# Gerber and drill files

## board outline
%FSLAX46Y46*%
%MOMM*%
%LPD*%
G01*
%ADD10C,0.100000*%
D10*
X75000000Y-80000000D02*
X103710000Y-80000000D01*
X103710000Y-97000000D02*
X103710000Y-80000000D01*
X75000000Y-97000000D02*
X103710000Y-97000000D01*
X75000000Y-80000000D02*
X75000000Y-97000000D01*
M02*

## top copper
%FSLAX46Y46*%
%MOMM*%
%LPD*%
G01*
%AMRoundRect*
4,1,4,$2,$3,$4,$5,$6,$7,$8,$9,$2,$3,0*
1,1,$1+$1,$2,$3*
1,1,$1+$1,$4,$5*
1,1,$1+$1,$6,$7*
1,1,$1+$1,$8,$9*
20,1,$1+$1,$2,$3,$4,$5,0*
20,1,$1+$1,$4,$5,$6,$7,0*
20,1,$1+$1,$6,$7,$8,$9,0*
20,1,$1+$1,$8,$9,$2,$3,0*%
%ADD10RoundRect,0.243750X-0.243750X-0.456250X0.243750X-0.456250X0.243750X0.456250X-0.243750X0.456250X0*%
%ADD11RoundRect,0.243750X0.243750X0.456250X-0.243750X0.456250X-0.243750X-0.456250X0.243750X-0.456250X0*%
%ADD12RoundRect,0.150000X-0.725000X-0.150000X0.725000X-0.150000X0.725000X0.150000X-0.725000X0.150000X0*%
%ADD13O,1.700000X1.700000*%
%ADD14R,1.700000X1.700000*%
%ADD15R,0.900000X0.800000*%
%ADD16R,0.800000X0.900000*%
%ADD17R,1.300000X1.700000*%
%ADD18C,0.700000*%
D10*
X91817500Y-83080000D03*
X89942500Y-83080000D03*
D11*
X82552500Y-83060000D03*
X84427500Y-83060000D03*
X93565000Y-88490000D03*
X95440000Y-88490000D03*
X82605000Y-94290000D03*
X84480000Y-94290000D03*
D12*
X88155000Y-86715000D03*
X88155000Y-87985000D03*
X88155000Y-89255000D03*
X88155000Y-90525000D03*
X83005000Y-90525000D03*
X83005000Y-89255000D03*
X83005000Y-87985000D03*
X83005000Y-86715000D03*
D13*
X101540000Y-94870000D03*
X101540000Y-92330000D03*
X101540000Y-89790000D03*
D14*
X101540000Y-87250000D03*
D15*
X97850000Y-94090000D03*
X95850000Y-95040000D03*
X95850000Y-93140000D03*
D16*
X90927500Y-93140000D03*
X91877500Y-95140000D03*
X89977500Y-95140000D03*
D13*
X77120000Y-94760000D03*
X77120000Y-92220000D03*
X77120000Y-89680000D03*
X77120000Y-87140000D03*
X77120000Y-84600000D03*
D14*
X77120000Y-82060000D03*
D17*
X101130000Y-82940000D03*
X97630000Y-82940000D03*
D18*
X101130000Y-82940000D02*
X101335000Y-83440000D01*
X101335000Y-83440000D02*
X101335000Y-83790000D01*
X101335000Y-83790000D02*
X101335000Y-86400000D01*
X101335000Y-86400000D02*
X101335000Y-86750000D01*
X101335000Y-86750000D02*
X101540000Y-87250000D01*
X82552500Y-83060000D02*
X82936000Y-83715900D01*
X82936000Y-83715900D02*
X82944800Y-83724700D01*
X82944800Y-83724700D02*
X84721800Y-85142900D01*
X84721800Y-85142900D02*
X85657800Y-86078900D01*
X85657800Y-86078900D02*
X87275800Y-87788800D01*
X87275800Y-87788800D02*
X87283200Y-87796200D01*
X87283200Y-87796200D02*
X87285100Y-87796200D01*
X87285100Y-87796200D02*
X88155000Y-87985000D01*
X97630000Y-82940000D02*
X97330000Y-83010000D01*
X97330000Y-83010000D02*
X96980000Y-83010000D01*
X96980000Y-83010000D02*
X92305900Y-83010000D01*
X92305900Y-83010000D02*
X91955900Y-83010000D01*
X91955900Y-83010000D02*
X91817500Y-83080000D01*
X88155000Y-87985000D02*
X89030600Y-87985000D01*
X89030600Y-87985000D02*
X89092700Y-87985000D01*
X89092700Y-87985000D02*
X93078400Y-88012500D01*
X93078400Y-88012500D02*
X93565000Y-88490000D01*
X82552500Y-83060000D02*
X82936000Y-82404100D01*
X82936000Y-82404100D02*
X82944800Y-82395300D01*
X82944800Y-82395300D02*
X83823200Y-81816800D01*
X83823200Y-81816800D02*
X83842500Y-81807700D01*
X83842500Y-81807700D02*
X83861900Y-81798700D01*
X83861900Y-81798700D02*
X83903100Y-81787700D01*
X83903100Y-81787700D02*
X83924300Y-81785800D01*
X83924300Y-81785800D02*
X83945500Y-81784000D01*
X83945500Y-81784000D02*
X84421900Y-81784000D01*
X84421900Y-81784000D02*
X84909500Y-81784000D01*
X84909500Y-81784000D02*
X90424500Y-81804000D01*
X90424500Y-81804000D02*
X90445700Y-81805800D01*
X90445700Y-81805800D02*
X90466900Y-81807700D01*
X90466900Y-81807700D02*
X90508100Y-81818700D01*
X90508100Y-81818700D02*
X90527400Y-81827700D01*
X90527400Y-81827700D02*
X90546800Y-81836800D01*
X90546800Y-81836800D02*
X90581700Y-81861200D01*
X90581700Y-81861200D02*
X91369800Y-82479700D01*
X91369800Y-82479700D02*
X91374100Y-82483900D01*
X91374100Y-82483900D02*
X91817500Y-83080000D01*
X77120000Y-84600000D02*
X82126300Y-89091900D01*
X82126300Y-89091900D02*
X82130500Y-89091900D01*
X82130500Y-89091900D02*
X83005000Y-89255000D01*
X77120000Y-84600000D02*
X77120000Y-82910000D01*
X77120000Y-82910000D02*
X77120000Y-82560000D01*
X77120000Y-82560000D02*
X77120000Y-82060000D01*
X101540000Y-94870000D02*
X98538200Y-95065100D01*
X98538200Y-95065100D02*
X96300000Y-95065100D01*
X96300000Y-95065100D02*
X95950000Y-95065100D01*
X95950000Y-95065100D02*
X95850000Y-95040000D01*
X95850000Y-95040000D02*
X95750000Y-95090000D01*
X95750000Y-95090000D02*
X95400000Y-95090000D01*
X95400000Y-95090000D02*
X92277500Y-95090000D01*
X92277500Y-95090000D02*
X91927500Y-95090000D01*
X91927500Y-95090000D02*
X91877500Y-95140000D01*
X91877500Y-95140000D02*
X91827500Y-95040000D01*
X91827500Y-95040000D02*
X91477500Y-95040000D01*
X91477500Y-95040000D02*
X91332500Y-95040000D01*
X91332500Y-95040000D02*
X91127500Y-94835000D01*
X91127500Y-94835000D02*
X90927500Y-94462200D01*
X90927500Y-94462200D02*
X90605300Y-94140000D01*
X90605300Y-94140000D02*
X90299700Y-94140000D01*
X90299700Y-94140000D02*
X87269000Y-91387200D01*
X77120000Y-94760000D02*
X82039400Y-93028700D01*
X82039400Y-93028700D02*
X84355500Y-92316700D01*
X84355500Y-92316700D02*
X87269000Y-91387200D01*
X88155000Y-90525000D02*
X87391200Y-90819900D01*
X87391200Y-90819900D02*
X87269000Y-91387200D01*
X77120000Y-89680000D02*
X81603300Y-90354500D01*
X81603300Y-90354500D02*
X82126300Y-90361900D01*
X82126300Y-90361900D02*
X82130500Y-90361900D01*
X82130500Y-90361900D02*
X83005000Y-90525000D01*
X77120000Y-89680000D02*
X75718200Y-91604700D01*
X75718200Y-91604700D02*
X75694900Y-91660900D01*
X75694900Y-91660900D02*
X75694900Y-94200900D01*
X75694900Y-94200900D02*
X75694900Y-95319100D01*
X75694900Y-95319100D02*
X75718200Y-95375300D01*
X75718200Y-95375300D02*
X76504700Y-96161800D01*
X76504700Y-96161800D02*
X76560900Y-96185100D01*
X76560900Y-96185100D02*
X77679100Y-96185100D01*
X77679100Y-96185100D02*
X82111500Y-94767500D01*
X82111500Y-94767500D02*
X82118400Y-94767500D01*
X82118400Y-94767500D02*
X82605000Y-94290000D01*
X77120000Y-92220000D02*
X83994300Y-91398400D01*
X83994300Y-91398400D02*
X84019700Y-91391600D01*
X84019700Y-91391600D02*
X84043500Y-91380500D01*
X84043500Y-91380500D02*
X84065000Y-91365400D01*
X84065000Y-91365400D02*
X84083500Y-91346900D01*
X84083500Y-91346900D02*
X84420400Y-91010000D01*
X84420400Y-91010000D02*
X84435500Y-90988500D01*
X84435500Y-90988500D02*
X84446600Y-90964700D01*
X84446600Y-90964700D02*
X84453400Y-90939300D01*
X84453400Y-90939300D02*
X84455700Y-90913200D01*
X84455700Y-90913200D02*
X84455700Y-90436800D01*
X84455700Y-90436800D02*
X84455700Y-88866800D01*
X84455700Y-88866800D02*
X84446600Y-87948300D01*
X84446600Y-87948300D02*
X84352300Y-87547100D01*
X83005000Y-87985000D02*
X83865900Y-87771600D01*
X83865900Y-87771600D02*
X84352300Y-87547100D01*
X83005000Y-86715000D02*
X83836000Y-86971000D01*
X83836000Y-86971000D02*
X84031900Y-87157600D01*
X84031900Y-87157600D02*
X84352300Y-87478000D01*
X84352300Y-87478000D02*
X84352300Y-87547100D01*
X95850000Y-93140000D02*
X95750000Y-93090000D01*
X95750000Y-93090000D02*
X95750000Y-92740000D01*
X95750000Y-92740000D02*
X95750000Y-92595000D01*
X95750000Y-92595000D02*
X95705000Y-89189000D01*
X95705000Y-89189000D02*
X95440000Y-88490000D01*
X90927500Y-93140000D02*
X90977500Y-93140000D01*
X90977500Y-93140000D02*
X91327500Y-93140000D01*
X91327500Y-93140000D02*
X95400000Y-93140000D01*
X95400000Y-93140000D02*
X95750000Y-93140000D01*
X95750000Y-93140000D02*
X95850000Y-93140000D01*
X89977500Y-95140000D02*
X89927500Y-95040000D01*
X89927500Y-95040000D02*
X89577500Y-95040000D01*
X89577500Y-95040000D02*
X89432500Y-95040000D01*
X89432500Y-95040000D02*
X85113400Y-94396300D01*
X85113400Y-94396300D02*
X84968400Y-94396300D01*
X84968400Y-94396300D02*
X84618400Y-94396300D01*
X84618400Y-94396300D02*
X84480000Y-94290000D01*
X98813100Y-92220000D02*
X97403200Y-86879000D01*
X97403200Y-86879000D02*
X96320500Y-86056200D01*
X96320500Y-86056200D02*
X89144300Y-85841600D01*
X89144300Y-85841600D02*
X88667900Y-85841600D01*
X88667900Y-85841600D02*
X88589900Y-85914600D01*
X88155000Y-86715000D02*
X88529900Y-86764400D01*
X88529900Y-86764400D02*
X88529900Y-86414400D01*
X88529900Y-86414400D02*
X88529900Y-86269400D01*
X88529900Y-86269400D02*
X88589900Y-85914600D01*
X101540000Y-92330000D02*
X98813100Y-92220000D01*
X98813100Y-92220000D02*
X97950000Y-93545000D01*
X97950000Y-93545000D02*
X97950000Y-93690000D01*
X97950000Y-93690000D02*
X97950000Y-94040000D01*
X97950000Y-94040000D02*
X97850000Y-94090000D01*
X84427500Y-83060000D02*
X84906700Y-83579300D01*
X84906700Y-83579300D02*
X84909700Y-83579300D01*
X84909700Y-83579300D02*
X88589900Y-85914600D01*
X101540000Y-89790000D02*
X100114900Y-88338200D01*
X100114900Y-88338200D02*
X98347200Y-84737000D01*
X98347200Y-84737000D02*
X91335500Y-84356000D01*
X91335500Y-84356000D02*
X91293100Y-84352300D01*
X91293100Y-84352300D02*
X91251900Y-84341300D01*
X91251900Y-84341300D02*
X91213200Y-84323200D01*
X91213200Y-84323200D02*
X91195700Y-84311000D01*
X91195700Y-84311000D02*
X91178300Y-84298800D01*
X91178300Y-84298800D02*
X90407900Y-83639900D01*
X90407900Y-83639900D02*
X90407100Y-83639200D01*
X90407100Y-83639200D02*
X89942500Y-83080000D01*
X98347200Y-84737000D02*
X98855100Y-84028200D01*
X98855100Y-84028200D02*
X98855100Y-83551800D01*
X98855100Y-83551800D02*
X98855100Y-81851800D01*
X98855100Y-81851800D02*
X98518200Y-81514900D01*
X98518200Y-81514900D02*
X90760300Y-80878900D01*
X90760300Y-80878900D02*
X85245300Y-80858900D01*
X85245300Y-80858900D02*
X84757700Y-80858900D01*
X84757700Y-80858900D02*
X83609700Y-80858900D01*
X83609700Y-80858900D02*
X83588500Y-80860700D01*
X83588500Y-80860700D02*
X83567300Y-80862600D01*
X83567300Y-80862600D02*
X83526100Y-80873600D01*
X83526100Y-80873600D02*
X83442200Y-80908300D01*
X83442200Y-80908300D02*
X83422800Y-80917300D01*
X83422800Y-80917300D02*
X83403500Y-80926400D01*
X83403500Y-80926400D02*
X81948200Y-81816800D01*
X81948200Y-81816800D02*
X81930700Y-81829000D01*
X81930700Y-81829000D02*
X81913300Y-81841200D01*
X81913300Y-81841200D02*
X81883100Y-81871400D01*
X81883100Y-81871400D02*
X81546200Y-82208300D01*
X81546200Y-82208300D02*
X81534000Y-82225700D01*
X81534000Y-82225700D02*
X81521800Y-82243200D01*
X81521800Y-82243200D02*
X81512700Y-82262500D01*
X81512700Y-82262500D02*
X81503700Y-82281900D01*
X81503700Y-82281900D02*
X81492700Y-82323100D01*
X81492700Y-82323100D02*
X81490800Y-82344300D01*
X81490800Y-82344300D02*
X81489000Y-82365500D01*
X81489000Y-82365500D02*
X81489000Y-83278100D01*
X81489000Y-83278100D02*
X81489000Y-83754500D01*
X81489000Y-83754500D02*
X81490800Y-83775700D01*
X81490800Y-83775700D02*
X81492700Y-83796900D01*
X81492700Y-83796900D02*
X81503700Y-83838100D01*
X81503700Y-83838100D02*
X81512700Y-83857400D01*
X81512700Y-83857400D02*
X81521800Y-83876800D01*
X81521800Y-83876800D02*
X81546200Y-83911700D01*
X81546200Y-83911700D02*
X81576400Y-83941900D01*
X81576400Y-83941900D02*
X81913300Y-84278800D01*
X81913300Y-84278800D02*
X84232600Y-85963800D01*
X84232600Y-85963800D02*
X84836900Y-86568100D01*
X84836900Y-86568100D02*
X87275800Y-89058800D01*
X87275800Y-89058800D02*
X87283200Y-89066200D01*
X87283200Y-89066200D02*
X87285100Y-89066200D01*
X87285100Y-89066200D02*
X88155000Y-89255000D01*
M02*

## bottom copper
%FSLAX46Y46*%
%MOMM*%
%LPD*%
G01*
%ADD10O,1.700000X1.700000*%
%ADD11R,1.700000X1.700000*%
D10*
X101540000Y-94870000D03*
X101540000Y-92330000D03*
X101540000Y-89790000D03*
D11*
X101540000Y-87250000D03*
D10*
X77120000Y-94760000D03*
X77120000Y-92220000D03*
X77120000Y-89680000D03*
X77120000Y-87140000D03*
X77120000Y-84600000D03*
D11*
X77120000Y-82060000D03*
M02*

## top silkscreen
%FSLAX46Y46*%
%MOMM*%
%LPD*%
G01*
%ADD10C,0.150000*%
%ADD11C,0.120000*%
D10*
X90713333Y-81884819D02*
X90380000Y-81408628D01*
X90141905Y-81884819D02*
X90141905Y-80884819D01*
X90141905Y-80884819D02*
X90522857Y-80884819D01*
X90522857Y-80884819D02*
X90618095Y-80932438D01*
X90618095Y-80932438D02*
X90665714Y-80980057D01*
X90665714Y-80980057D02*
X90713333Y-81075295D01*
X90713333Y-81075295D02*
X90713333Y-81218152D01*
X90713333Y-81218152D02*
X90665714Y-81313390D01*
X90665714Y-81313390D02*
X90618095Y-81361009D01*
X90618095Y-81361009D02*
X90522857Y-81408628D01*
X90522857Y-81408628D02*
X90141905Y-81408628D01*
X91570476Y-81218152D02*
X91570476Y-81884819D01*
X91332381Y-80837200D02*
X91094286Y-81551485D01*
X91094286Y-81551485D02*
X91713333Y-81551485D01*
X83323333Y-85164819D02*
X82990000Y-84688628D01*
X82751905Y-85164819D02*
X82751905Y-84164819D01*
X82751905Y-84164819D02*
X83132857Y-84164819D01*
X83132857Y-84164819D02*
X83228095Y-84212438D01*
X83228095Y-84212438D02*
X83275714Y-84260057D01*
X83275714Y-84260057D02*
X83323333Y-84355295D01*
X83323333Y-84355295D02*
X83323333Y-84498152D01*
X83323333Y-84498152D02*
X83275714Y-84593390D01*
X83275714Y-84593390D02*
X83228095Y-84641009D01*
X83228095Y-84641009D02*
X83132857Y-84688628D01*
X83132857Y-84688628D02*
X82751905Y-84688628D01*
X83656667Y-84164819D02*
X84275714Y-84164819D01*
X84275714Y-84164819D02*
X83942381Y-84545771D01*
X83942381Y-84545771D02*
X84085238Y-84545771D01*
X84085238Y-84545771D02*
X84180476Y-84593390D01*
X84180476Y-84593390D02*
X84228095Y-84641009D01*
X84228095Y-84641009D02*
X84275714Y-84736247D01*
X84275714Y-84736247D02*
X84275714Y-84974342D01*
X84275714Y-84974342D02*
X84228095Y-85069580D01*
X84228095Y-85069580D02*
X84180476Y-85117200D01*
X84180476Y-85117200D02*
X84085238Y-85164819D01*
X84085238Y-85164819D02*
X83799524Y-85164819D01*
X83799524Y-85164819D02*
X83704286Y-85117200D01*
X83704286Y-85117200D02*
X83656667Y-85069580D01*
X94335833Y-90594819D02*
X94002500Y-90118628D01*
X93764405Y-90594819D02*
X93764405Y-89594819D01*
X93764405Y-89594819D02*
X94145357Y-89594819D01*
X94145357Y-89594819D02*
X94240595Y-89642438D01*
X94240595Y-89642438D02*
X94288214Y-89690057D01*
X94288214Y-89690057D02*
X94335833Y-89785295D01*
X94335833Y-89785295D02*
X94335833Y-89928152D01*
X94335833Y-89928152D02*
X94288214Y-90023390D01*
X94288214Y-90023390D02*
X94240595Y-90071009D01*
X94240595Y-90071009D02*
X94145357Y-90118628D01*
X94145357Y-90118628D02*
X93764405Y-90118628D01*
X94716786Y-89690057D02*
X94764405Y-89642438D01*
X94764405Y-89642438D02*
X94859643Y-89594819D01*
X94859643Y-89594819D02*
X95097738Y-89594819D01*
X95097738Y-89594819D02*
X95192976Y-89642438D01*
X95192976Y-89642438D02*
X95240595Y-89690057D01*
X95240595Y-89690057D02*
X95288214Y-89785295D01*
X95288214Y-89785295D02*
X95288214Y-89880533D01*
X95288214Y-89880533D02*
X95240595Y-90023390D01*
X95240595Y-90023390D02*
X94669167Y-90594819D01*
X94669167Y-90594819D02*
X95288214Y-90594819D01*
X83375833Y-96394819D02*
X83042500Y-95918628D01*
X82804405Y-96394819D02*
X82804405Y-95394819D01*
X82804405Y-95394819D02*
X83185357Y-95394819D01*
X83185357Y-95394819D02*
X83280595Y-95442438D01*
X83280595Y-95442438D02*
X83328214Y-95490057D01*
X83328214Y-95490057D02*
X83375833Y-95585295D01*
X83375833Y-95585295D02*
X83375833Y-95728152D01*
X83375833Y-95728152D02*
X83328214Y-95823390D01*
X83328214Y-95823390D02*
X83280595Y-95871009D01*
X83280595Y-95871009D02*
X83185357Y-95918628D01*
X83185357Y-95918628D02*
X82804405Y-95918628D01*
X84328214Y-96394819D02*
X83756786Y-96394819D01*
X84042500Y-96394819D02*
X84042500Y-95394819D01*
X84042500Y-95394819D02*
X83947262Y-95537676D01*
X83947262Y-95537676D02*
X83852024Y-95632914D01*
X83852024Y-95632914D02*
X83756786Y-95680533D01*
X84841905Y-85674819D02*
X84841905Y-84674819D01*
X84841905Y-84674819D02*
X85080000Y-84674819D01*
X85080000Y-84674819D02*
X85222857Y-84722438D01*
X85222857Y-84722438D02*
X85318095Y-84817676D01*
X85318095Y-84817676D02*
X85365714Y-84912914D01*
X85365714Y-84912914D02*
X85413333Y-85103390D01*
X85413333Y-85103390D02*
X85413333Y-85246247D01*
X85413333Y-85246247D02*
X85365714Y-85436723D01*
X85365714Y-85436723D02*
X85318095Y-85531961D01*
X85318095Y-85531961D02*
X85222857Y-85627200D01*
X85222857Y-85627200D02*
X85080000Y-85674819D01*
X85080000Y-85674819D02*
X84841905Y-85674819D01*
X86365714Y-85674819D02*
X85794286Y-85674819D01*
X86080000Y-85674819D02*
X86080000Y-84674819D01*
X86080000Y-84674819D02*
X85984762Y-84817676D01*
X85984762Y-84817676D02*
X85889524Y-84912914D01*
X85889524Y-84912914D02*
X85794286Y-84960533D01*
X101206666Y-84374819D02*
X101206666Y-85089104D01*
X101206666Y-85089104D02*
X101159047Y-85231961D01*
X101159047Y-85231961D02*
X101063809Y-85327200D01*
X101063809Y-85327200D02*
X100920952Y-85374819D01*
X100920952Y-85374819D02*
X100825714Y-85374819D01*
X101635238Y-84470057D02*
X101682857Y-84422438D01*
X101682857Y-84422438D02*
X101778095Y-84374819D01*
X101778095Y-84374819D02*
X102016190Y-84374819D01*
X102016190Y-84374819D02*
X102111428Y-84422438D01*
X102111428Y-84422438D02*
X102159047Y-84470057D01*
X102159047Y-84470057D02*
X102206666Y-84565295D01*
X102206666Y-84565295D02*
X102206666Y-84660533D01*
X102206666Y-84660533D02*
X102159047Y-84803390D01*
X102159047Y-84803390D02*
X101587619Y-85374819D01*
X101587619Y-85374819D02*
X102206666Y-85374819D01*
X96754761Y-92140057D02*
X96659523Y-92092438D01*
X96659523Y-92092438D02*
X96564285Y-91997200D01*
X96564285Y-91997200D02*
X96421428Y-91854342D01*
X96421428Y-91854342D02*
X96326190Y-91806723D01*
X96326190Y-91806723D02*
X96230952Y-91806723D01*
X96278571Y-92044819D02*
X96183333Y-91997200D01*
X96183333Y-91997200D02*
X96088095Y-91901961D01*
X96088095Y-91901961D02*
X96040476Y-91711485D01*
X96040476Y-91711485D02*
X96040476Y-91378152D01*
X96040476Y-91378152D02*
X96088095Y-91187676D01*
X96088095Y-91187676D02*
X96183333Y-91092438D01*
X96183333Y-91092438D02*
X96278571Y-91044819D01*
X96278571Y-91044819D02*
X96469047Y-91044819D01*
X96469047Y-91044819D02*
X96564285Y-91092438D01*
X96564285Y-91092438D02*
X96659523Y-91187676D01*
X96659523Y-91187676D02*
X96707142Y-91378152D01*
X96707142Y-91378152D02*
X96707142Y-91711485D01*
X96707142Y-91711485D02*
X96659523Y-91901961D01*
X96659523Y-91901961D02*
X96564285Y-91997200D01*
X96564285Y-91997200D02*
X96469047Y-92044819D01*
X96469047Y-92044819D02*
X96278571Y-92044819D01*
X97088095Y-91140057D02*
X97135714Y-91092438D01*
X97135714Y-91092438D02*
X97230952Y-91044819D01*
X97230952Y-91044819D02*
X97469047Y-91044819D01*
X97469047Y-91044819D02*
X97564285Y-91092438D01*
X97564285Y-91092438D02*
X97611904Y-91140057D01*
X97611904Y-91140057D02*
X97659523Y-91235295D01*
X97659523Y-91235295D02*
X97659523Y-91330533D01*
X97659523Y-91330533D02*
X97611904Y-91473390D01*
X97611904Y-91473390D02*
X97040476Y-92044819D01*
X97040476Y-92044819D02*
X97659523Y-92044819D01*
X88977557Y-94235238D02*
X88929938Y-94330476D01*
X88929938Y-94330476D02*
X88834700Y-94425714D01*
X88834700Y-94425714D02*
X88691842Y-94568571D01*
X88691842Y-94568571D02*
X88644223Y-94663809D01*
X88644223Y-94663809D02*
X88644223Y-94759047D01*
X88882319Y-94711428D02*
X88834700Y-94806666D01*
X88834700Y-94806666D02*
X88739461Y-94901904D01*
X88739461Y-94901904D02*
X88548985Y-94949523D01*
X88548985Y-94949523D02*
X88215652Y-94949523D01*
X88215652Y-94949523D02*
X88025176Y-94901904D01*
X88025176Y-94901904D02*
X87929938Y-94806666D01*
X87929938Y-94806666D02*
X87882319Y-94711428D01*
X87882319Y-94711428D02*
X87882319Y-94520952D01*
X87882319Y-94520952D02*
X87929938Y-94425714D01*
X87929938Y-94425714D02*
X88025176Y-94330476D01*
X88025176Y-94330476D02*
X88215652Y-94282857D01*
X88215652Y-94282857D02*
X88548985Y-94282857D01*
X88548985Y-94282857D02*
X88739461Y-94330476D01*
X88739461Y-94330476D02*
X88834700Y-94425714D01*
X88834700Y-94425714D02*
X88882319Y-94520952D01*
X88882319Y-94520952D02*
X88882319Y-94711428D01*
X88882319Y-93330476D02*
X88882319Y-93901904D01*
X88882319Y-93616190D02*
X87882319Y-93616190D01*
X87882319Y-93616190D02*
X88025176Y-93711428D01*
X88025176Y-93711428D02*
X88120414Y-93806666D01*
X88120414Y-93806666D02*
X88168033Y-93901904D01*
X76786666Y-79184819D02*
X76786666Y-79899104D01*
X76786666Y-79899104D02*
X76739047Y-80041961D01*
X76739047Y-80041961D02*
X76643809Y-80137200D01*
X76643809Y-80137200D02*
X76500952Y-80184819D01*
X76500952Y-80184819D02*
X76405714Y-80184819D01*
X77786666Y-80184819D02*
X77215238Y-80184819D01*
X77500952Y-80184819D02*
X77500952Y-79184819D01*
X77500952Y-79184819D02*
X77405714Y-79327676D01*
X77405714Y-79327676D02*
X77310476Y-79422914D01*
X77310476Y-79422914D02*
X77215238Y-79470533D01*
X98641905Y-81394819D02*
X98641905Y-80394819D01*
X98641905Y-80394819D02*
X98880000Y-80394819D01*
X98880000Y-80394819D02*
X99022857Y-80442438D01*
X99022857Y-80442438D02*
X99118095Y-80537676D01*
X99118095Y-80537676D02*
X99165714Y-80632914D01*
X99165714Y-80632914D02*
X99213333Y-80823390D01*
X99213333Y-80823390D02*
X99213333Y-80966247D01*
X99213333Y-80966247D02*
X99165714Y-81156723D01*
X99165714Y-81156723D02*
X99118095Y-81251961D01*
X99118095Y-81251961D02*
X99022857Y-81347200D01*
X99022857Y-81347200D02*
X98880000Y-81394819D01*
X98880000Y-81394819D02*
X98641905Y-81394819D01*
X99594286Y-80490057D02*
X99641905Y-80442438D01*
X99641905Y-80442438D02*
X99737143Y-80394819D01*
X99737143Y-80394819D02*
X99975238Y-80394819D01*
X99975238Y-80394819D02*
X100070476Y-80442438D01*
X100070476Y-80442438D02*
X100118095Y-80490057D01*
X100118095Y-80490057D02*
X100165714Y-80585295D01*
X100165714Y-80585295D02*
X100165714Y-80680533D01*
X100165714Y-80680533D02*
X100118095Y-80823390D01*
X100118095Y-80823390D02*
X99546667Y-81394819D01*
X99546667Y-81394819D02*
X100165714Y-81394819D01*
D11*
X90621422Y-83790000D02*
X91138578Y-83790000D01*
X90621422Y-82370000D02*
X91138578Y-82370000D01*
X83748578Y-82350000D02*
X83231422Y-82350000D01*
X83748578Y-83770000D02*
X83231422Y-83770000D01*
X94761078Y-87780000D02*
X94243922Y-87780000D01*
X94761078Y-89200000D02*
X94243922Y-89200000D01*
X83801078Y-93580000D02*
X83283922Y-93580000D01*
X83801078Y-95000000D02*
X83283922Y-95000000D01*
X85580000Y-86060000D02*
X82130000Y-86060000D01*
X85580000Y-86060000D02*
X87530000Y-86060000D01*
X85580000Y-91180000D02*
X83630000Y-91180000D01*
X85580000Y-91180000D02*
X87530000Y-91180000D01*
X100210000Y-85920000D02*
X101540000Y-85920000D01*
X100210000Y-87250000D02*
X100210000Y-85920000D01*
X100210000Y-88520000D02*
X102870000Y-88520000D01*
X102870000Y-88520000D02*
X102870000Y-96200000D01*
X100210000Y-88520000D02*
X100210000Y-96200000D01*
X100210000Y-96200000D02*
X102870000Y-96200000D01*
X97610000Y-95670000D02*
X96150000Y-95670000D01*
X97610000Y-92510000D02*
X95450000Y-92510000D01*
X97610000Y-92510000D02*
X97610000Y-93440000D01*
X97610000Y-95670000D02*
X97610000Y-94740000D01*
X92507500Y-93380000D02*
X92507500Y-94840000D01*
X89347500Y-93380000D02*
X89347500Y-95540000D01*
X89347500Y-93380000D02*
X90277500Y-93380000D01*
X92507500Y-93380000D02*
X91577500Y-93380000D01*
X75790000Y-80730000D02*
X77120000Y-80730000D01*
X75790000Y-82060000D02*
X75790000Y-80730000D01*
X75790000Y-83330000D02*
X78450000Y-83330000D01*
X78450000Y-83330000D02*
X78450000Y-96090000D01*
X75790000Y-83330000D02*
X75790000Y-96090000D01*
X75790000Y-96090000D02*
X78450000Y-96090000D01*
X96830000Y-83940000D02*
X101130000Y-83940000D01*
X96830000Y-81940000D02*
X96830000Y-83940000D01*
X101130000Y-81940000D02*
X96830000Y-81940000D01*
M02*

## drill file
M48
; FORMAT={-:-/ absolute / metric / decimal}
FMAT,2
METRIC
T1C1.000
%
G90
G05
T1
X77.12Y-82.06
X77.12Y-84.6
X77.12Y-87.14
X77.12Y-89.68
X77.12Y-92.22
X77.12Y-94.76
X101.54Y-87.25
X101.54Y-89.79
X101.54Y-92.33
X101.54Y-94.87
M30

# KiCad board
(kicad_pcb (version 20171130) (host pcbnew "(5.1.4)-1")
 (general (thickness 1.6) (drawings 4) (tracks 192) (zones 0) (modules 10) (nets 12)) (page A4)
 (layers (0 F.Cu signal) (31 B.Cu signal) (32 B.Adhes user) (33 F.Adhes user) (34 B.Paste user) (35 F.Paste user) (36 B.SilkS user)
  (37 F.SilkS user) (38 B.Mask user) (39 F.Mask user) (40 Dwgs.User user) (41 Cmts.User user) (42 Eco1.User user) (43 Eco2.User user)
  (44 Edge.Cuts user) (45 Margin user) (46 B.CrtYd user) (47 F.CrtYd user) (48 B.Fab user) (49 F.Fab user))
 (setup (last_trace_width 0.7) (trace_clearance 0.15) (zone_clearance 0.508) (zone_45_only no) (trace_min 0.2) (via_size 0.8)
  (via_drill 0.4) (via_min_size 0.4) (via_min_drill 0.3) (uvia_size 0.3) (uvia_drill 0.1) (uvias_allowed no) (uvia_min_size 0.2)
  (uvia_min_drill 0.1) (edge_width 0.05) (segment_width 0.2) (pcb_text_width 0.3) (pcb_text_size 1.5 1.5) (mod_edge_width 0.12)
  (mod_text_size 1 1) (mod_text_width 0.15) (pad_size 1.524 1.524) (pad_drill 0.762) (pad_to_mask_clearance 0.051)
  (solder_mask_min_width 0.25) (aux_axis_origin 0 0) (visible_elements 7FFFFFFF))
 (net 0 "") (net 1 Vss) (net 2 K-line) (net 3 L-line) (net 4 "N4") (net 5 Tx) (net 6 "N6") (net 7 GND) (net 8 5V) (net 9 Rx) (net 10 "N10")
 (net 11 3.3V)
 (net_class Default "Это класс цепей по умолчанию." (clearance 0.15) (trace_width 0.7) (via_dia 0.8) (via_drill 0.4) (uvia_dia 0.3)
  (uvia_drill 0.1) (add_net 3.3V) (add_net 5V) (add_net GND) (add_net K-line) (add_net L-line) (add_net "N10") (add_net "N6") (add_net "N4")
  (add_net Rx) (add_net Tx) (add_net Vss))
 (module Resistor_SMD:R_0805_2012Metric (layer F.Cu) (at 90.88 83.08)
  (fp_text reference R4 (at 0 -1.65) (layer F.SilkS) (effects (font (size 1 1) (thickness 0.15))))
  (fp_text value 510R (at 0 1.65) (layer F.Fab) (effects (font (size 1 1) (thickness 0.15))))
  (fp_line (start -0.258578 0.71) (end 0.258578 0.71) (layer F.SilkS) (width 0.12))
  (fp_line (start -0.258578 -0.71) (end 0.258578 -0.71) (layer F.SilkS) (width 0.12))
  (pad 2 smd roundrect (at 0.9375 0) (size 0.975 1.4) (layers F.Cu F.Paste F.Mask) (roundrect_rratio 0.25) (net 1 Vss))
  (pad 1 smd roundrect (at -0.9375 0) (size 0.975 1.4) (layers F.Cu F.Paste F.Mask) (roundrect_rratio 0.25) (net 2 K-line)))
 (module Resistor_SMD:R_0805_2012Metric (layer F.Cu) (at 83.49 83.06 180)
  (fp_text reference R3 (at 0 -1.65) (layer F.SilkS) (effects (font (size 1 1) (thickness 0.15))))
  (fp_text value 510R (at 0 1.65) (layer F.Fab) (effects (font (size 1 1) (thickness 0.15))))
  (fp_line (start -0.258578 0.71) (end 0.258578 0.71) (layer F.SilkS) (width 0.12))
  (fp_line (start -0.258578 -0.71) (end 0.258578 -0.71) (layer F.SilkS) (width 0.12))
  (pad 2 smd roundrect (at 0.9375 0 180) (size 0.975 1.4) (layers F.Cu F.Paste F.Mask) (roundrect_rratio 0.25) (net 1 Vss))
  (pad 1 smd roundrect (at -0.9375 0 180) (size 0.975 1.4) (layers F.Cu F.Paste F.Mask) (roundrect_rratio 0.25) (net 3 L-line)))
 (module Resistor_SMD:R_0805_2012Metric (layer F.Cu) (at 94.5025 88.49 180)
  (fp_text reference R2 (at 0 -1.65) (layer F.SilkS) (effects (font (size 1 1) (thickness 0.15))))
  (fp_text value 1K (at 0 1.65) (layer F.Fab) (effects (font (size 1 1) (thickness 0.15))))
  (fp_line (start -0.258578 0.71) (end 0.258578 0.71) (layer F.SilkS) (width 0.12))
  (fp_line (start -0.258578 -0.71) (end 0.258578 -0.71) (layer F.SilkS) (width 0.12))
  (pad 2 smd roundrect (at 0.9375 0 180) (size 0.975 1.4) (layers F.Cu F.Paste F.Mask) (roundrect_rratio 0.25) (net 1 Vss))
  (pad 1 smd roundrect (at -0.9375 0 180) (size 0.975 1.4) (layers F.Cu F.Paste F.Mask) (roundrect_rratio 0.25) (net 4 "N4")))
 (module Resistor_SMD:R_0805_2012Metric (layer F.Cu) (at 83.5425 94.29 180)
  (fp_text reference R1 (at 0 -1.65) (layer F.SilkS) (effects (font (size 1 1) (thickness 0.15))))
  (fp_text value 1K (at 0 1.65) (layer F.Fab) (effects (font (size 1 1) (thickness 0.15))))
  (fp_line (start -0.258578 0.71) (end 0.258578 0.71) (layer F.SilkS) (width 0.12))
  (fp_line (start -0.258578 -0.71) (end 0.258578 -0.71) (layer F.SilkS) (width 0.12))
  (pad 2 smd roundrect (at 0.9375 0 180) (size 0.975 1.4) (layers F.Cu F.Paste F.Mask) (roundrect_rratio 0.25) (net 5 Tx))
  (pad 1 smd roundrect (at -0.9375 0 180) (size 0.975 1.4) (layers F.Cu F.Paste F.Mask) (roundrect_rratio 0.25) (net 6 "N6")))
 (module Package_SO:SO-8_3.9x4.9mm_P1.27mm (layer F.Cu) (at 85.58 88.62)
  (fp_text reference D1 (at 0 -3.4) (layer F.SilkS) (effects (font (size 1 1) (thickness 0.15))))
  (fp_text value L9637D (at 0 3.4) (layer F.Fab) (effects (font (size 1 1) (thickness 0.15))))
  (fp_line (start 0 -2.56) (end -3.45 -2.56) (layer F.SilkS) (width 0.12))
  (fp_line (start 0 -2.56) (end 1.95 -2.56) (layer F.SilkS) (width 0.12))
  (fp_line (start 0 2.56) (end -1.95 2.56) (layer F.SilkS) (width 0.12))
  (fp_line (start 0 2.56) (end 1.95 2.56) (layer F.SilkS) (width 0.12))
  (pad 8 smd roundrect (at 2.575 -1.905) (size 1.75 0.6) (layers F.Cu F.Paste F.Mask) (roundrect_rratio 0.25) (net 3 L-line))
  (pad 7 smd roundrect (at 2.575 -0.635) (size 1.75 0.6) (layers F.Cu F.Paste F.Mask) (roundrect_rratio 0.25) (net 1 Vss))
  (pad 6 smd roundrect (at 2.575 0.635) (size 1.75 0.6) (layers F.Cu F.Paste F.Mask) (roundrect_rratio 0.25) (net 2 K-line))
  (pad 5 smd roundrect (at 2.575 1.905) (size 1.75 0.6) (layers F.Cu F.Paste F.Mask) (roundrect_rratio 0.25) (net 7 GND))
  (pad 4 smd roundrect (at -2.575 1.905) (size 1.75 0.6) (layers F.Cu F.Paste F.Mask) (roundrect_rratio 0.25) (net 5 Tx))
  (pad 3 smd roundrect (at -2.575 0.635) (size 1.75 0.6) (layers F.Cu F.Paste F.Mask) (roundrect_rratio 0.25) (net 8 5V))
  (pad 2 smd roundrect (at -2.575 -0.635) (size 1.75 0.6) (layers F.Cu F.Paste F.Mask) (roundrect_rratio 0.25) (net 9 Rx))
  (pad 1 smd roundrect (at -2.575 -1.905) (size 1.75 0.6) (layers F.Cu F.Paste F.Mask) (roundrect_rratio 0.25) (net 9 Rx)))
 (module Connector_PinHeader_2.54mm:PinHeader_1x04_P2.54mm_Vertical (layer F.Cu) (at 101.54 87.25)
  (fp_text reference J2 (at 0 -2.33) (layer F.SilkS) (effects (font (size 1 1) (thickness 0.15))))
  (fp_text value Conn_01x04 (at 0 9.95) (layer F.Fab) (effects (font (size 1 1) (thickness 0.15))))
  (fp_line (start -1.33 -1.33) (end 0 -1.33) (layer F.SilkS) (width 0.12))
  (fp_line (start -1.33 0) (end -1.33 -1.33) (layer F.SilkS) (width 0.12))
  (fp_line (start -1.33 1.27) (end 1.33 1.27) (layer F.SilkS) (width 0.12))
  (fp_line (start 1.33 1.27) (end 1.33 8.95) (layer F.SilkS) (width 0.12))
  (fp_line (start -1.33 1.27) (end -1.33 8.95) (layer F.SilkS) (width 0.12))
  (fp_line (start -1.33 8.95) (end 1.33 8.95) (layer F.SilkS) (width 0.12))
  (pad 4 thru_hole oval (at 0 7.62) (size 1.7 1.7) (drill 1) (layers *.Cu *.Mask) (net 7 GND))
  (pad 3 thru_hole oval (at 0 5.08) (size 1.7 1.7) (drill 1) (layers *.Cu *.Mask) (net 3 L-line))
  (pad 2 thru_hole oval (at 0 2.54) (size 1.7 1.7) (drill 1) (layers *.Cu *.Mask) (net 2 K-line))
  (pad 1 thru_hole rect (at 0 0) (size 1.7 1.7) (drill 1) (layers *.Cu *.Mask) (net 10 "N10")))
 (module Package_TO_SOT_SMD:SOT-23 (layer F.Cu) (at 96.85 94.09)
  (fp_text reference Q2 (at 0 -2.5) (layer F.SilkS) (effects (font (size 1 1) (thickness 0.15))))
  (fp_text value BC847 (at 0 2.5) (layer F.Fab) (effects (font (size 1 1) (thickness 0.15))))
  (fp_line (start 0.76 1.58) (end -0.7 1.58) (layer F.SilkS) (width 0.12))
  (fp_line (start 0.76 -1.58) (end -1.4 -1.58) (layer F.SilkS) (width 0.12))
  (fp_line (start 0.76 -1.58) (end 0.76 -0.65) (layer F.SilkS) (width 0.12))
  (fp_line (start 0.76 1.58) (end 0.76 0.65) (layer F.SilkS) (width 0.12))
  (pad 3 smd rect (at 1 0) (size 0.9 0.8) (layers F.Cu F.Paste F.Mask) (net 3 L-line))
  (pad 2 smd rect (at -1 0.95) (size 0.9 0.8) (layers F.Cu F.Paste F.Mask) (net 7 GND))
  (pad 1 smd rect (at -1 -0.95) (size 0.9 0.8) (layers F.Cu F.Paste F.Mask) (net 4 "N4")))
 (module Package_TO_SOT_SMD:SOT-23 (layer F.Cu) (at 90.9275 94.14 90)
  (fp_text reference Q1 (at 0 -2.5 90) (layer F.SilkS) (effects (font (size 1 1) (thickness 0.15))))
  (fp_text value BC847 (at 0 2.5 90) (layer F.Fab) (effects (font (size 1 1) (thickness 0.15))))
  (fp_line (start 0.76 1.58) (end -0.7 1.58) (layer F.SilkS) (width 0.12))
  (fp_line (start 0.76 -1.58) (end -1.4 -1.58) (layer F.SilkS) (width 0.12))
  (fp_line (start 0.76 -1.58) (end 0.76 -0.65) (layer F.SilkS) (width 0.12))
  (fp_line (start 0.76 1.58) (end 0.76 0.65) (layer F.SilkS) (width 0.12))
  (pad 3 smd rect (at 1 0 90) (size 0.9 0.8) (layers F.Cu F.Paste F.Mask) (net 4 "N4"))
  (pad 2 smd rect (at -1 0.95 90) (size 0.9 0.8) (layers F.Cu F.Paste F.Mask) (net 7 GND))
  (pad 1 smd rect (at -1 -0.95 90) (size 0.9 0.8) (layers F.Cu F.Paste F.Mask) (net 6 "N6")))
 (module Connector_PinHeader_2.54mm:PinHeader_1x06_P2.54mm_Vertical (layer F.Cu) (at 77.12 82.06)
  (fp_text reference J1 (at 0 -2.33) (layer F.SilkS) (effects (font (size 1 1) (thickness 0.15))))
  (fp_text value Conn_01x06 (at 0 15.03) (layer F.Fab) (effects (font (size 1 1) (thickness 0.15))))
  (fp_line (start -1.33 -1.33) (end 0 -1.33) (layer F.SilkS) (width 0.12))
  (fp_line (start -1.33 0) (end -1.33 -1.33) (layer F.SilkS) (width 0.12))
  (fp_line (start -1.33 1.27) (end 1.33 1.27) (layer F.SilkS) (width 0.12))
  (fp_line (start 1.33 1.27) (end 1.33 14.03) (layer F.SilkS) (width 0.12))
  (fp_line (start -1.33 1.27) (end -1.33 14.03) (layer F.SilkS) (width 0.12))
  (fp_line (start -1.33 14.03) (end 1.33 14.03) (layer F.SilkS) (width 0.12))
  (pad 6 thru_hole oval (at 0 12.7) (size 1.7 1.7) (drill 1) (layers *.Cu *.Mask) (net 7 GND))
  (pad 5 thru_hole oval (at 0 10.16) (size 1.7 1.7) (drill 1) (layers *.Cu *.Mask) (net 9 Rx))
  (pad 4 thru_hole oval (at 0 7.62) (size 1.7 1.7) (drill 1) (layers *.Cu *.Mask) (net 5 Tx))
  (pad 3 thru_hole oval (at 0 5.08) (size 1.7 1.7) (drill 1) (layers *.Cu *.Mask) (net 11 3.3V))
  (pad 2 thru_hole oval (at 0 2.54) (size 1.7 1.7) (drill 1) (layers *.Cu *.Mask) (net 8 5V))
  (pad 1 thru_hole rect (at 0 0) (size 1.7 1.7) (drill 1) (layers *.Cu *.Mask) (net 8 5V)))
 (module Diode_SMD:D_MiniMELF (layer F.Cu) (at 99.38 82.94)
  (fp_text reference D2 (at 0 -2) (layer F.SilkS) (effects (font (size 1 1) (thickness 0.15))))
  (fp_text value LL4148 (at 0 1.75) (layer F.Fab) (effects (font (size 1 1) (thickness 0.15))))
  (fp_line (start -2.55 1) (end 1.75 1) (layer F.SilkS) (width 0.12))
  (fp_line (start -2.55 -1) (end -2.55 1) (layer F.SilkS) (width 0.12))
  (fp_line (start 1.75 -1) (end -2.55 -1) (layer F.SilkS) (width 0.12))
  (pad 2 smd rect (at 1.75 0) (size 1.3 1.7) (layers F.Cu F.Paste F.Mask) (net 10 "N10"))
  (pad 1 smd rect (at -1.75 0) (size 1.3 1.7) (layers F.Cu F.Paste F.Mask) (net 1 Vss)))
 (gr_line (start 75 80) (end 103.71 80) (layer Edge.Cuts) (width 0.1))
 (gr_line (start 103.71 97) (end 103.71 80) (layer Edge.Cuts) (width 0.1))
 (gr_line (start 75 97) (end 103.71 97) (layer Edge.Cuts) (width 0.1))
 (gr_line (start 75 80) (end 75 97) (layer Edge.Cuts) (width 0.1))
 (segment (start 101.13 82.94) (end 101.335 83.44) (width 0.7) (layer F.Cu) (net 10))
 (segment (start 101.335 83.44) (end 101.335 83.79) (width 0.7) (layer F.Cu) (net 10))
 (segment (start 101.335 83.79) (end 101.335 86.4) (width 0.7) (layer F.Cu) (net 10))
 (segment (start 101.335 86.4) (end 101.335 86.75) (width 0.7) (layer F.Cu) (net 10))
 (segment (start 101.335 86.75) (end 101.54 87.25) (width 0.7) (layer F.Cu) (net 10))
 (segment (start 82.5525 83.06) (end 82.936 83.7159) (width 0.7) (layer F.Cu) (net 1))
 (segment (start 82.936 83.7159) (end 82.9448 83.7247) (width 0.7) (layer F.Cu) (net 1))
 (segment (start 82.9448 83.7247) (end 84.7218 85.1429) (width 0.7) (layer F.Cu) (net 1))
 (segment (start 84.7218 85.1429) (end 85.6578 86.0789) (width 0.7) (layer F.Cu) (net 1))
 (segment (start 85.6578 86.0789) (end 87.2758 87.7888) (width 0.7) (layer F.Cu) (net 1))
 (segment (start 87.2758 87.7888) (end 87.2832 87.7962) (width 0.7) (layer F.Cu) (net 1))
 (segment (start 87.2832 87.7962) (end 87.2851 87.7962) (width 0.7) (layer F.Cu) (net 1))
 (segment (start 87.2851 87.7962) (end 88.155 87.985) (width 0.7) (layer F.Cu) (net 1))
 (segment (start 97.63 82.94) (end 97.33 83.01) (width 0.7) (layer F.Cu) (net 1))
 (segment (start 97.33 83.01) (end 96.98 83.01) (width 0.7) (layer F.Cu) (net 1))
 (segment (start 96.98 83.01) (end 92.3059 83.01) (width 0.7) (layer F.Cu) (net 1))
 (segment (start 92.3059 83.01) (end 91.9559 83.01) (width 0.7) (layer F.Cu) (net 1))
 (segment (start 91.9559 83.01) (end 91.8175 83.08) (width 0.7) (layer F.Cu) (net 1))
 (segment (start 88.155 87.985) (end 89.0306 87.985) (width 0.7) (layer F.Cu) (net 1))
 (segment (start 89.0306 87.985) (end 89.0927 87.985) (width 0.7) (layer F.Cu) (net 1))
 (segment (start 89.0927 87.985) (end 93.0784 88.0125) (width 0.7) (layer F.Cu) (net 1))
 (segment (start 93.0784 88.0125) (end 93.565 88.49) (width 0.7) (layer F.Cu) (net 1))
 (segment (start 82.5525 83.06) (end 82.936 82.4041) (width 0.7) (layer F.Cu) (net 1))
 (segment (start 82.936 82.4041) (end 82.9448 82.3953) (width 0.7) (layer F.Cu) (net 1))
 (segment (start 82.9448 82.3953) (end 83.8232 81.8168) (width 0.7) (layer F.Cu) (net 1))
 (segment (start 83.8232 81.8168) (end 83.8425 81.8077) (width 0.7) (layer F.Cu) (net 1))
 (segment (start 83.8425 81.8077) (end 83.8619 81.7987) (width 0.7) (layer F.Cu) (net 1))
 (segment (start 83.8619 81.7987) (end 83.9031 81.7877) (width 0.7) (layer F.Cu) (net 1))
 (segment (start 83.9031 81.7877) (end 83.9243 81.7858) (width 0.7) (layer F.Cu) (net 1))
 (segment (start 83.9243 81.7858) (end 83.9455 81.784) (width 0.7) (layer F.Cu) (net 1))
 (segment (start 83.9455 81.784) (end 84.4219 81.784) (width 0.7) (layer F.Cu) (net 1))
 (segment (start 84.4219 81.784) (end 84.9095 81.784) (width 0.7) (layer F.Cu) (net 1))
 (segment (start 84.9095 81.784) (end 90.4245 81.804) (width 0.7) (layer F.Cu) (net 1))
 (segment (start 90.4245 81.804) (end 90.4457 81.8058) (width 0.7) (layer F.Cu) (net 1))
 (segment (start 90.4457 81.8058) (end 90.4669 81.8077) (width 0.7) (layer F.Cu) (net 1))
 (segment (start 90.4669 81.8077) (end 90.5081 81.8187) (width 0.7) (layer F.Cu) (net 1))
 (segment (start 90.5081 81.8187) (end 90.5274 81.8277) (width 0.7) (layer F.Cu) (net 1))
 (segment (start 90.5274 81.8277) (end 90.5468 81.8368) (width 0.7) (layer F.Cu) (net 1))
 (segment (start 90.5468 81.8368) (end 90.5817 81.8612) (width 0.7) (layer F.Cu) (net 1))
 (segment (start 90.5817 81.8612) (end 91.3698 82.4797) (width 0.7) (layer F.Cu) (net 1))
 (segment (start 91.3698 82.4797) (end 91.3741 82.4839) (width 0.7) (layer F.Cu) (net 1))
 (segment (start 91.3741 82.4839) (end 91.8175 83.08) (width 0.7) (layer F.Cu) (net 1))
 (segment (start 77.12 84.6) (end 82.1263 89.0919) (width 0.7) (layer F.Cu) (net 8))
 (segment (start 82.1263 89.0919) (end 82.1305 89.0919) (width 0.7) (layer F.Cu) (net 8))
 (segment (start 82.1305 89.0919) (end 83.005 89.255) (width 0.7) (layer F.Cu) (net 8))
 (segment (start 77.12 84.6) (end 77.12 82.91) (width 0.7) (layer F.Cu) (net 8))
 (segment (start 77.12 82.91) (end 77.12 82.56) (width 0.7) (layer F.Cu) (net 8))
 (segment (start 77.12 82.56) (end 77.12 82.06) (width 0.7) (layer F.Cu) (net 8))
 (segment (start 101.54 94.87) (end 98.5382 95.0651) (width 0.7) (layer F.Cu) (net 7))
 (segment (start 98.5382 95.0651) (end 96.3 95.0651) (width 0.7) (layer F.Cu) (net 7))
 (segment (start 96.3 95.0651) (end 95.95 95.0651) (width 0.7) (layer F.Cu) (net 7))
 (segment (start 95.95 95.0651) (end 95.85 95.04) (width 0.7) (layer F.Cu) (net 7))
 (segment (start 95.85 95.04) (end 95.75 95.09) (width 0.7) (layer F.Cu) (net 7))
 (segment (start 95.75 95.09) (end 95.4 95.09) (width 0.7) (layer F.Cu) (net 7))
 (segment (start 95.4 95.09) (end 92.2775 95.09) (width 0.7) (layer F.Cu) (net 7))
 (segment (start 92.2775 95.09) (end 91.9275 95.09) (width 0.7) (layer F.Cu) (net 7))
 (segment (start 91.9275 95.09) (end 91.8775 95.14) (width 0.7) (layer F.Cu) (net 7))
 (segment (start 91.8775 95.14) (end 91.8275 95.04) (width 0.7) (layer F.Cu) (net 7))
 (segment (start 91.8275 95.04) (end 91.4775 95.04) (width 0.7) (layer F.Cu) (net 7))
 (segment (start 91.4775 95.04) (end 91.3325 95.04) (width 0.7) (layer F.Cu) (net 7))
 (segment (start 91.3325 95.04) (end 91.1275 94.835) (width 0.7) (layer F.Cu) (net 7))
 (segment (start 91.1275 94.835) (end 90.9275 94.4622) (width 0.7) (layer F.Cu) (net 7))
 (segment (start 90.9275 94.4622) (end 90.6053 94.14) (width 0.7) (layer F.Cu) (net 7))
 (segment (start 90.6053 94.14) (end 90.2997 94.14) (width 0.7) (layer F.Cu) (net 7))
 (segment (start 90.2997 94.14) (end 87.269 91.3872) (width 0.7) (layer F.Cu) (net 7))
 (segment (start 77.12 94.76) (end 82.0394 93.0287) (width 0.7) (layer F.Cu) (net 7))
 (segment (start 82.0394 93.0287) (end 84.3555 92.3167) (width 0.7) (layer F.Cu) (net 7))
 (segment (start 84.3555 92.3167) (end 87.269 91.3872) (width 0.7) (layer F.Cu) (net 7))
 (segment (start 88.155 90.525) (end 87.3912 90.8199) (width 0.7) (layer F.Cu) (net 7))
 (segment (start 87.3912 90.8199) (end 87.269 91.3872) (width 0.7) (layer F.Cu) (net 7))
 (segment (start 77.12 89.68) (end 81.6033 90.3545) (width 0.7) (layer F.Cu) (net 5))
 (segment (start 81.6033 90.3545) (end 82.1263 90.3619) (width 0.7) (layer F.Cu) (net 5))
 (segment (start 82.1263 90.3619) (end 82.1305 90.3619) (width 0.7) (layer F.Cu) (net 5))
 (segment (start 82.1305 90.3619) (end 83.005 90.525) (width 0.7) (layer F.Cu) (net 5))
 (segment (start 77.12 89.68) (end 75.7182 91.6047) (width 0.7) (layer F.Cu) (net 5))
 (segment (start 75.7182 91.6047) (end 75.6949 91.6609) (width 0.7) (layer F.Cu) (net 5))
 (segment (start 75.6949 91.6609) (end 75.6949 94.2009) (width 0.7) (layer F.Cu) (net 5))
 (segment (start 75.6949 94.2009) (end 75.6949 95.3191) (width 0.7) (layer F.Cu) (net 5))
 (segment (start 75.6949 95.3191) (end 75.7182 95.3753) (width 0.7) (layer F.Cu) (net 5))
 (segment (start 75.7182 95.3753) (end 76.5047 96.1618) (width 0.7) (layer F.Cu) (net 5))
 (segment (start 76.5047 96.1618) (end 76.5609 96.1851) (width 0.7) (layer F.Cu) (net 5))
 (segment (start 76.5609 96.1851) (end 77.6791 96.1851) (width 0.7) (layer F.Cu) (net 5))
 (segment (start 77.6791 96.1851) (end 82.1115 94.7675) (width 0.7) (layer F.Cu) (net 5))
 (segment (start 82.1115 94.7675) (end 82.1184 94.7675) (width 0.7) (layer F.Cu) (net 5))
 (segment (start 82.1184 94.7675) (end 82.605 94.29) (width 0.7) (layer F.Cu) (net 5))
 (segment (start 77.12 92.22) (end 83.9943 91.3984) (width 0.7) (layer F.Cu) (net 9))
 (segment (start 83.9943 91.3984) (end 84.0197 91.3916) (width 0.7) (layer F.Cu) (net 9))
 (segment (start 84.0197 91.3916) (end 84.0435 91.3805) (width 0.7) (layer F.Cu) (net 9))
 (segment (start 84.0435 91.3805) (end 84.065 91.3654) (width 0.7) (layer F.Cu) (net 9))
 (segment (start 84.065 91.3654) (end 84.0835 91.3469) (width 0.7) (layer F.Cu) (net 9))
 (segment (start 84.0835 91.3469) (end 84.4204 91.01) (width 0.7) (layer F.Cu) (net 9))
 (segment (start 84.4204 91.01) (end 84.4355 90.9885) (width 0.7) (layer F.Cu) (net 9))
 (segment (start 84.4355 90.9885) (end 84.4466 90.9647) (width 0.7) (layer F.Cu) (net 9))
 (segment (start 84.4466 90.9647) (end 84.4534 90.9393) (width 0.7) (layer F.Cu) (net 9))
 (segment (start 84.4534 90.9393) (end 84.4557 90.9132) (width 0.7) (layer F.Cu) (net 9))
 (segment (start 84.4557 90.9132) (end 84.4557 90.4368) (width 0.7) (layer F.Cu) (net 9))
 (segment (start 84.4557 90.4368) (end 84.4557 88.8668) (width 0.7) (layer F.Cu) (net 9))
 (segment (start 84.4557 88.8668) (end 84.4466 87.9483) (width 0.7) (layer F.Cu) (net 9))
 (segment (start 84.4466 87.9483) (end 84.3523 87.5471) (width 0.7) (layer F.Cu) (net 9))
 (segment (start 83.005 87.985) (end 83.8659 87.7716) (width 0.7) (layer F.Cu) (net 9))
 (segment (start 83.8659 87.7716) (end 84.3523 87.5471) (width 0.7) (layer F.Cu) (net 9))
 (segment (start 83.005 86.715) (end 83.836 86.971) (width 0.7) (layer F.Cu) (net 9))
 (segment (start 83.836 86.971) (end 84.0319 87.1576) (width 0.7) (layer F.Cu) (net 9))
 (segment (start 84.0319 87.1576) (end 84.3523 87.478) (width 0.7) (layer F.Cu) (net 9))
 (segment (start 84.3523 87.478) (end 84.3523 87.5471) (width 0.7) (layer F.Cu) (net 9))
 (segment (start 95.85 93.14) (end 95.75 93.09) (width 0.7) (layer F.Cu) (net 4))
 (segment (start 95.75 93.09) (end 95.75 92.74) (width 0.7) (layer F.Cu) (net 4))
 (segment (start 95.75 92.74) (end 95.75 92.595) (width 0.7) (layer F.Cu) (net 4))
 (segment (start 95.75 92.595) (end 95.705 89.189) (width 0.7) (layer F.Cu) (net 4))
 (segment (start 95.705 89.189) (end 95.44 88.49) (width 0.7) (layer F.Cu) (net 4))
 (segment (start 90.9275 93.14) (end 90.9775 93.14) (width 0.7) (layer F.Cu) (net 4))
 (segment (start 90.9775 93.14) (end 91.3275 93.14) (width 0.7) (layer F.Cu) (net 4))
 (segment (start 91.3275 93.14) (end 95.4 93.14) (width 0.7) (layer F.Cu) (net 4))
 (segment (start 95.4 93.14) (end 95.75 93.14) (width 0.7) (layer F.Cu) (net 4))
 (segment (start 95.75 93.14) (end 95.85 93.14) (width 0.7) (layer F.Cu) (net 4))
 (segment (start 89.9775 95.14) (end 89.9275 95.04) (width 0.7) (layer F.Cu) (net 6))
 (segment (start 89.9275 95.04) (end 89.5775 95.04) (width 0.7) (layer F.Cu) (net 6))
 (segment (start 89.5775 95.04) (end 89.4325 95.04) (width 0.7) (layer F.Cu) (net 6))
 (segment (start 89.4325 95.04) (end 85.1134 94.3963) (width 0.7) (layer F.Cu) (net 6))
 (segment (start 85.1134 94.3963) (end 84.9684 94.3963) (width 0.7) (layer F.Cu) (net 6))
 (segment (start 84.9684 94.3963) (end 84.6184 94.3963) (width 0.7) (layer F.Cu) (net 6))
 (segment (start 84.6184 94.3963) (end 84.48 94.29) (width 0.7) (layer F.Cu) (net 6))
 (segment (start 98.8131 92.22) (end 97.4032 86.879) (width 0.7) (layer F.Cu) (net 3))
 (segment (start 97.4032 86.879) (end 96.3205 86.0562) (width 0.7) (layer F.Cu) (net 3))
 (segment (start 96.3205 86.0562) (end 89.1443 85.8416) (width 0.7) (layer F.Cu) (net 3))
 (segment (start 89.1443 85.8416) (end 88.6679 85.8416) (width 0.7) (layer F.Cu) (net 3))
 (segment (start 88.6679 85.8416) (end 88.5899 85.9146) (width 0.7) (layer F.Cu) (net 3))
 (segment (start 88.155 86.715) (end 88.5299 86.7644) (width 0.7) (layer F.Cu) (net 3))
 (segment (start 88.5299 86.7644) (end 88.5299 86.4144) (width 0.7) (layer F.Cu) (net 3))
 (segment (start 88.5299 86.4144) (end 88.5299 86.2694) (width 0.7) (layer F.Cu) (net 3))
 (segment (start 88.5299 86.2694) (end 88.5899 85.9146) (width 0.7) (layer F.Cu) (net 3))
 (segment (start 101.54 92.33) (end 98.8131 92.22) (width 0.7) (layer F.Cu) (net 3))
 (segment (start 98.8131 92.22) (end 97.95 93.545) (width 0.7) (layer F.Cu) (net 3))
 (segment (start 97.95 93.545) (end 97.95 93.69) (width 0.7) (layer F.Cu) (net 3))
 (segment (start 97.95 93.69) (end 97.95 94.04) (width 0.7) (layer F.Cu) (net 3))
 (segment (start 97.95 94.04) (end 97.85 94.09) (width 0.7) (layer F.Cu) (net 3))
 (segment (start 84.4275 83.06) (end 84.9067 83.5793) (width 0.7) (layer F.Cu) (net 3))
 (segment (start 84.9067 83.5793) (end 84.9097 83.5793) (width 0.7) (layer F.Cu) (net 3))
 (segment (start 84.9097 83.5793) (end 88.5899 85.9146) (width 0.7) (layer F.Cu) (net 3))
 (segment (start 101.54 89.79) (end 100.1149 88.3382) (width 0.7) (layer F.Cu) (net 2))
 (segment (start 100.1149 88.3382) (end 98.3472 84.737) (width 0.7) (layer F.Cu) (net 2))
 (segment (start 98.3472 84.737) (end 91.3355 84.356) (width 0.7) (layer F.Cu) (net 2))
 (segment (start 91.3355 84.356) (end 91.2931 84.3523) (width 0.7) (layer F.Cu) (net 2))
 (segment (start 91.2931 84.3523) (end 91.2519 84.3413) (width 0.7) (layer F.Cu) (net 2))
 (segment (start 91.2519 84.3413) (end 91.2132 84.3232) (width 0.7) (layer F.Cu) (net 2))
 (segment (start 91.2132 84.3232) (end 91.1957 84.311) (width 0.7) (layer F.Cu) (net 2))
 (segment (start 91.1957 84.311) (end 91.1783 84.2988) (width 0.7) (layer F.Cu) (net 2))
 (segment (start 91.1783 84.2988) (end 90.4079 83.6399) (width 0.7) (layer F.Cu) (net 2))
 (segment (start 90.4079 83.6399) (end 90.4071 83.6392) (width 0.7) (layer F.Cu) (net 2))
 (segment (start 90.4071 83.6392) (end 89.9425 83.08) (width 0.7) (layer F.Cu) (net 2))
 (segment (start 98.3472 84.737) (end 98.8551 84.0282) (width 0.7) (layer F.Cu) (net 2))
 (segment (start 98.8551 84.0282) (end 98.8551 83.5518) (width 0.7) (layer F.Cu) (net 2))
 (segment (start 98.8551 83.5518) (end 98.8551 81.8518) (width 0.7) (layer F.Cu) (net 2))
 (segment (start 98.8551 81.8518) (end 98.5182 81.5149) (width 0.7) (layer F.Cu) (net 2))
 (segment (start 98.5182 81.5149) (end 90.7603 80.8789) (width 0.7) (layer F.Cu) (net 2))
 (segment (start 90.7603 80.8789) (end 85.2453 80.8589) (width 0.7) (layer F.Cu) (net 2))
 (segment (start 85.2453 80.8589) (end 84.7577 80.8589) (width 0.7) (layer F.Cu) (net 2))
 (segment (start 84.7577 80.8589) (end 83.6097 80.8589) (width 0.7) (layer F.Cu) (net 2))
 (segment (start 83.6097 80.8589) (end 83.5885 80.8607) (width 0.7) (layer F.Cu) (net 2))
 (segment (start 83.5885 80.8607) (end 83.5673 80.8626) (width 0.7) (layer F.Cu) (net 2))
 (segment (start 83.5673 80.8626) (end 83.5261 80.8736) (width 0.7) (layer F.Cu) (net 2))
 (segment (start 83.5261 80.8736) (end 83.4422 80.9083) (width 0.7) (layer F.Cu) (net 2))
 (segment (start 83.4422 80.9083) (end 83.4228 80.9173) (width 0.7) (layer F.Cu) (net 2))
 (segment (start 83.4228 80.9173) (end 83.4035 80.9264) (width 0.7) (layer F.Cu) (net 2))
 (segment (start 83.4035 80.9264) (end 81.9482 81.8168) (width 0.7) (layer F.Cu) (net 2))
 (segment (start 81.9482 81.8168) (end 81.9307 81.829) (width 0.7) (layer F.Cu) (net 2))
 (segment (start 81.9307 81.829) (end 81.9133 81.8412) (width 0.7) (layer F.Cu) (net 2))
 (segment (start 81.9133 81.8412) (end 81.8831 81.8714) (width 0.7) (layer F.Cu) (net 2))
 (segment (start 81.8831 81.8714) (end 81.5462 82.2083) (width 0.7) (layer F.Cu) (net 2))
 (segment (start 81.5462 82.2083) (end 81.534 82.2257) (width 0.7) (layer F.Cu) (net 2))
 (segment (start 81.534 82.2257) (end 81.5218 82.2432) (width 0.7) (layer F.Cu) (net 2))
 (segment (start 81.5218 82.2432) (end 81.5127 82.2625) (width 0.7) (layer F.Cu) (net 2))
 (segment (start 81.5127 82.2625) (end 81.5037 82.2819) (width 0.7) (layer F.Cu) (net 2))
 (segment (start 81.5037 82.2819) (end 81.4927 82.3231) (width 0.7) (layer F.Cu) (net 2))
 (segment (start 81.4927 82.3231) (end 81.4908 82.3443) (width 0.7) (layer F.Cu) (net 2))
 (segment (start 81.4908 82.3443) (end 81.489 82.3655) (width 0.7) (layer F.Cu) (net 2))
 (segment (start 81.489 82.3655) (end 81.489 83.2781) (width 0.7) (layer F.Cu) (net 2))
 (segment (start 81.489 83.2781) (end 81.489 83.7545) (width 0.7) (layer F.Cu) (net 2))
 (segment (start 81.489 83.7545) (end 81.4908 83.7757) (width 0.7) (layer F.Cu) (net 2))
 (segment (start 81.4908 83.7757) (end 81.4927 83.7969) (width 0.7) (layer F.Cu) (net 2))
 (segment (start 81.4927 83.7969) (end 81.5037 83.8381) (width 0.7) (layer F.Cu) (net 2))
 (segment (start 81.5037 83.8381) (end 81.5127 83.8574) (width 0.7) (layer F.Cu) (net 2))
 (segment (start 81.5127 83.8574) (end 81.5218 83.8768) (width 0.7) (layer F.Cu) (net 2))
 (segment (start 81.5218 83.8768) (end 81.5462 83.9117) (width 0.7) (layer F.Cu) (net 2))
 (segment (start 81.5462 83.9117) (end 81.5764 83.9419) (width 0.7) (layer F.Cu) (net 2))
 (segment (start 81.5764 83.9419) (end 81.9133 84.2788) (width 0.7) (layer F.Cu) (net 2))
 (segment (start 81.9133 84.2788) (end 84.2326 85.9638) (width 0.7) (layer F.Cu) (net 2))
 (segment (start 84.2326 85.9638) (end 84.8369 86.5681) (width 0.7) (layer F.Cu) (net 2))
 (segment (start 84.8369 86.5681) (end 87.2758 89.0588) (width 0.7) (layer F.Cu) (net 2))
 (segment (start 87.2758 89.0588) (end 87.2832 89.0662) (width 0.7) (layer F.Cu) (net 2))
 (segment (start 87.2832 89.0662) (end 87.2851 89.0662) (width 0.7) (layer F.Cu) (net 2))
 (segment (start 87.2851 89.0662) (end 88.155 89.255) (width 0.7) (layer F.Cu) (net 2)))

